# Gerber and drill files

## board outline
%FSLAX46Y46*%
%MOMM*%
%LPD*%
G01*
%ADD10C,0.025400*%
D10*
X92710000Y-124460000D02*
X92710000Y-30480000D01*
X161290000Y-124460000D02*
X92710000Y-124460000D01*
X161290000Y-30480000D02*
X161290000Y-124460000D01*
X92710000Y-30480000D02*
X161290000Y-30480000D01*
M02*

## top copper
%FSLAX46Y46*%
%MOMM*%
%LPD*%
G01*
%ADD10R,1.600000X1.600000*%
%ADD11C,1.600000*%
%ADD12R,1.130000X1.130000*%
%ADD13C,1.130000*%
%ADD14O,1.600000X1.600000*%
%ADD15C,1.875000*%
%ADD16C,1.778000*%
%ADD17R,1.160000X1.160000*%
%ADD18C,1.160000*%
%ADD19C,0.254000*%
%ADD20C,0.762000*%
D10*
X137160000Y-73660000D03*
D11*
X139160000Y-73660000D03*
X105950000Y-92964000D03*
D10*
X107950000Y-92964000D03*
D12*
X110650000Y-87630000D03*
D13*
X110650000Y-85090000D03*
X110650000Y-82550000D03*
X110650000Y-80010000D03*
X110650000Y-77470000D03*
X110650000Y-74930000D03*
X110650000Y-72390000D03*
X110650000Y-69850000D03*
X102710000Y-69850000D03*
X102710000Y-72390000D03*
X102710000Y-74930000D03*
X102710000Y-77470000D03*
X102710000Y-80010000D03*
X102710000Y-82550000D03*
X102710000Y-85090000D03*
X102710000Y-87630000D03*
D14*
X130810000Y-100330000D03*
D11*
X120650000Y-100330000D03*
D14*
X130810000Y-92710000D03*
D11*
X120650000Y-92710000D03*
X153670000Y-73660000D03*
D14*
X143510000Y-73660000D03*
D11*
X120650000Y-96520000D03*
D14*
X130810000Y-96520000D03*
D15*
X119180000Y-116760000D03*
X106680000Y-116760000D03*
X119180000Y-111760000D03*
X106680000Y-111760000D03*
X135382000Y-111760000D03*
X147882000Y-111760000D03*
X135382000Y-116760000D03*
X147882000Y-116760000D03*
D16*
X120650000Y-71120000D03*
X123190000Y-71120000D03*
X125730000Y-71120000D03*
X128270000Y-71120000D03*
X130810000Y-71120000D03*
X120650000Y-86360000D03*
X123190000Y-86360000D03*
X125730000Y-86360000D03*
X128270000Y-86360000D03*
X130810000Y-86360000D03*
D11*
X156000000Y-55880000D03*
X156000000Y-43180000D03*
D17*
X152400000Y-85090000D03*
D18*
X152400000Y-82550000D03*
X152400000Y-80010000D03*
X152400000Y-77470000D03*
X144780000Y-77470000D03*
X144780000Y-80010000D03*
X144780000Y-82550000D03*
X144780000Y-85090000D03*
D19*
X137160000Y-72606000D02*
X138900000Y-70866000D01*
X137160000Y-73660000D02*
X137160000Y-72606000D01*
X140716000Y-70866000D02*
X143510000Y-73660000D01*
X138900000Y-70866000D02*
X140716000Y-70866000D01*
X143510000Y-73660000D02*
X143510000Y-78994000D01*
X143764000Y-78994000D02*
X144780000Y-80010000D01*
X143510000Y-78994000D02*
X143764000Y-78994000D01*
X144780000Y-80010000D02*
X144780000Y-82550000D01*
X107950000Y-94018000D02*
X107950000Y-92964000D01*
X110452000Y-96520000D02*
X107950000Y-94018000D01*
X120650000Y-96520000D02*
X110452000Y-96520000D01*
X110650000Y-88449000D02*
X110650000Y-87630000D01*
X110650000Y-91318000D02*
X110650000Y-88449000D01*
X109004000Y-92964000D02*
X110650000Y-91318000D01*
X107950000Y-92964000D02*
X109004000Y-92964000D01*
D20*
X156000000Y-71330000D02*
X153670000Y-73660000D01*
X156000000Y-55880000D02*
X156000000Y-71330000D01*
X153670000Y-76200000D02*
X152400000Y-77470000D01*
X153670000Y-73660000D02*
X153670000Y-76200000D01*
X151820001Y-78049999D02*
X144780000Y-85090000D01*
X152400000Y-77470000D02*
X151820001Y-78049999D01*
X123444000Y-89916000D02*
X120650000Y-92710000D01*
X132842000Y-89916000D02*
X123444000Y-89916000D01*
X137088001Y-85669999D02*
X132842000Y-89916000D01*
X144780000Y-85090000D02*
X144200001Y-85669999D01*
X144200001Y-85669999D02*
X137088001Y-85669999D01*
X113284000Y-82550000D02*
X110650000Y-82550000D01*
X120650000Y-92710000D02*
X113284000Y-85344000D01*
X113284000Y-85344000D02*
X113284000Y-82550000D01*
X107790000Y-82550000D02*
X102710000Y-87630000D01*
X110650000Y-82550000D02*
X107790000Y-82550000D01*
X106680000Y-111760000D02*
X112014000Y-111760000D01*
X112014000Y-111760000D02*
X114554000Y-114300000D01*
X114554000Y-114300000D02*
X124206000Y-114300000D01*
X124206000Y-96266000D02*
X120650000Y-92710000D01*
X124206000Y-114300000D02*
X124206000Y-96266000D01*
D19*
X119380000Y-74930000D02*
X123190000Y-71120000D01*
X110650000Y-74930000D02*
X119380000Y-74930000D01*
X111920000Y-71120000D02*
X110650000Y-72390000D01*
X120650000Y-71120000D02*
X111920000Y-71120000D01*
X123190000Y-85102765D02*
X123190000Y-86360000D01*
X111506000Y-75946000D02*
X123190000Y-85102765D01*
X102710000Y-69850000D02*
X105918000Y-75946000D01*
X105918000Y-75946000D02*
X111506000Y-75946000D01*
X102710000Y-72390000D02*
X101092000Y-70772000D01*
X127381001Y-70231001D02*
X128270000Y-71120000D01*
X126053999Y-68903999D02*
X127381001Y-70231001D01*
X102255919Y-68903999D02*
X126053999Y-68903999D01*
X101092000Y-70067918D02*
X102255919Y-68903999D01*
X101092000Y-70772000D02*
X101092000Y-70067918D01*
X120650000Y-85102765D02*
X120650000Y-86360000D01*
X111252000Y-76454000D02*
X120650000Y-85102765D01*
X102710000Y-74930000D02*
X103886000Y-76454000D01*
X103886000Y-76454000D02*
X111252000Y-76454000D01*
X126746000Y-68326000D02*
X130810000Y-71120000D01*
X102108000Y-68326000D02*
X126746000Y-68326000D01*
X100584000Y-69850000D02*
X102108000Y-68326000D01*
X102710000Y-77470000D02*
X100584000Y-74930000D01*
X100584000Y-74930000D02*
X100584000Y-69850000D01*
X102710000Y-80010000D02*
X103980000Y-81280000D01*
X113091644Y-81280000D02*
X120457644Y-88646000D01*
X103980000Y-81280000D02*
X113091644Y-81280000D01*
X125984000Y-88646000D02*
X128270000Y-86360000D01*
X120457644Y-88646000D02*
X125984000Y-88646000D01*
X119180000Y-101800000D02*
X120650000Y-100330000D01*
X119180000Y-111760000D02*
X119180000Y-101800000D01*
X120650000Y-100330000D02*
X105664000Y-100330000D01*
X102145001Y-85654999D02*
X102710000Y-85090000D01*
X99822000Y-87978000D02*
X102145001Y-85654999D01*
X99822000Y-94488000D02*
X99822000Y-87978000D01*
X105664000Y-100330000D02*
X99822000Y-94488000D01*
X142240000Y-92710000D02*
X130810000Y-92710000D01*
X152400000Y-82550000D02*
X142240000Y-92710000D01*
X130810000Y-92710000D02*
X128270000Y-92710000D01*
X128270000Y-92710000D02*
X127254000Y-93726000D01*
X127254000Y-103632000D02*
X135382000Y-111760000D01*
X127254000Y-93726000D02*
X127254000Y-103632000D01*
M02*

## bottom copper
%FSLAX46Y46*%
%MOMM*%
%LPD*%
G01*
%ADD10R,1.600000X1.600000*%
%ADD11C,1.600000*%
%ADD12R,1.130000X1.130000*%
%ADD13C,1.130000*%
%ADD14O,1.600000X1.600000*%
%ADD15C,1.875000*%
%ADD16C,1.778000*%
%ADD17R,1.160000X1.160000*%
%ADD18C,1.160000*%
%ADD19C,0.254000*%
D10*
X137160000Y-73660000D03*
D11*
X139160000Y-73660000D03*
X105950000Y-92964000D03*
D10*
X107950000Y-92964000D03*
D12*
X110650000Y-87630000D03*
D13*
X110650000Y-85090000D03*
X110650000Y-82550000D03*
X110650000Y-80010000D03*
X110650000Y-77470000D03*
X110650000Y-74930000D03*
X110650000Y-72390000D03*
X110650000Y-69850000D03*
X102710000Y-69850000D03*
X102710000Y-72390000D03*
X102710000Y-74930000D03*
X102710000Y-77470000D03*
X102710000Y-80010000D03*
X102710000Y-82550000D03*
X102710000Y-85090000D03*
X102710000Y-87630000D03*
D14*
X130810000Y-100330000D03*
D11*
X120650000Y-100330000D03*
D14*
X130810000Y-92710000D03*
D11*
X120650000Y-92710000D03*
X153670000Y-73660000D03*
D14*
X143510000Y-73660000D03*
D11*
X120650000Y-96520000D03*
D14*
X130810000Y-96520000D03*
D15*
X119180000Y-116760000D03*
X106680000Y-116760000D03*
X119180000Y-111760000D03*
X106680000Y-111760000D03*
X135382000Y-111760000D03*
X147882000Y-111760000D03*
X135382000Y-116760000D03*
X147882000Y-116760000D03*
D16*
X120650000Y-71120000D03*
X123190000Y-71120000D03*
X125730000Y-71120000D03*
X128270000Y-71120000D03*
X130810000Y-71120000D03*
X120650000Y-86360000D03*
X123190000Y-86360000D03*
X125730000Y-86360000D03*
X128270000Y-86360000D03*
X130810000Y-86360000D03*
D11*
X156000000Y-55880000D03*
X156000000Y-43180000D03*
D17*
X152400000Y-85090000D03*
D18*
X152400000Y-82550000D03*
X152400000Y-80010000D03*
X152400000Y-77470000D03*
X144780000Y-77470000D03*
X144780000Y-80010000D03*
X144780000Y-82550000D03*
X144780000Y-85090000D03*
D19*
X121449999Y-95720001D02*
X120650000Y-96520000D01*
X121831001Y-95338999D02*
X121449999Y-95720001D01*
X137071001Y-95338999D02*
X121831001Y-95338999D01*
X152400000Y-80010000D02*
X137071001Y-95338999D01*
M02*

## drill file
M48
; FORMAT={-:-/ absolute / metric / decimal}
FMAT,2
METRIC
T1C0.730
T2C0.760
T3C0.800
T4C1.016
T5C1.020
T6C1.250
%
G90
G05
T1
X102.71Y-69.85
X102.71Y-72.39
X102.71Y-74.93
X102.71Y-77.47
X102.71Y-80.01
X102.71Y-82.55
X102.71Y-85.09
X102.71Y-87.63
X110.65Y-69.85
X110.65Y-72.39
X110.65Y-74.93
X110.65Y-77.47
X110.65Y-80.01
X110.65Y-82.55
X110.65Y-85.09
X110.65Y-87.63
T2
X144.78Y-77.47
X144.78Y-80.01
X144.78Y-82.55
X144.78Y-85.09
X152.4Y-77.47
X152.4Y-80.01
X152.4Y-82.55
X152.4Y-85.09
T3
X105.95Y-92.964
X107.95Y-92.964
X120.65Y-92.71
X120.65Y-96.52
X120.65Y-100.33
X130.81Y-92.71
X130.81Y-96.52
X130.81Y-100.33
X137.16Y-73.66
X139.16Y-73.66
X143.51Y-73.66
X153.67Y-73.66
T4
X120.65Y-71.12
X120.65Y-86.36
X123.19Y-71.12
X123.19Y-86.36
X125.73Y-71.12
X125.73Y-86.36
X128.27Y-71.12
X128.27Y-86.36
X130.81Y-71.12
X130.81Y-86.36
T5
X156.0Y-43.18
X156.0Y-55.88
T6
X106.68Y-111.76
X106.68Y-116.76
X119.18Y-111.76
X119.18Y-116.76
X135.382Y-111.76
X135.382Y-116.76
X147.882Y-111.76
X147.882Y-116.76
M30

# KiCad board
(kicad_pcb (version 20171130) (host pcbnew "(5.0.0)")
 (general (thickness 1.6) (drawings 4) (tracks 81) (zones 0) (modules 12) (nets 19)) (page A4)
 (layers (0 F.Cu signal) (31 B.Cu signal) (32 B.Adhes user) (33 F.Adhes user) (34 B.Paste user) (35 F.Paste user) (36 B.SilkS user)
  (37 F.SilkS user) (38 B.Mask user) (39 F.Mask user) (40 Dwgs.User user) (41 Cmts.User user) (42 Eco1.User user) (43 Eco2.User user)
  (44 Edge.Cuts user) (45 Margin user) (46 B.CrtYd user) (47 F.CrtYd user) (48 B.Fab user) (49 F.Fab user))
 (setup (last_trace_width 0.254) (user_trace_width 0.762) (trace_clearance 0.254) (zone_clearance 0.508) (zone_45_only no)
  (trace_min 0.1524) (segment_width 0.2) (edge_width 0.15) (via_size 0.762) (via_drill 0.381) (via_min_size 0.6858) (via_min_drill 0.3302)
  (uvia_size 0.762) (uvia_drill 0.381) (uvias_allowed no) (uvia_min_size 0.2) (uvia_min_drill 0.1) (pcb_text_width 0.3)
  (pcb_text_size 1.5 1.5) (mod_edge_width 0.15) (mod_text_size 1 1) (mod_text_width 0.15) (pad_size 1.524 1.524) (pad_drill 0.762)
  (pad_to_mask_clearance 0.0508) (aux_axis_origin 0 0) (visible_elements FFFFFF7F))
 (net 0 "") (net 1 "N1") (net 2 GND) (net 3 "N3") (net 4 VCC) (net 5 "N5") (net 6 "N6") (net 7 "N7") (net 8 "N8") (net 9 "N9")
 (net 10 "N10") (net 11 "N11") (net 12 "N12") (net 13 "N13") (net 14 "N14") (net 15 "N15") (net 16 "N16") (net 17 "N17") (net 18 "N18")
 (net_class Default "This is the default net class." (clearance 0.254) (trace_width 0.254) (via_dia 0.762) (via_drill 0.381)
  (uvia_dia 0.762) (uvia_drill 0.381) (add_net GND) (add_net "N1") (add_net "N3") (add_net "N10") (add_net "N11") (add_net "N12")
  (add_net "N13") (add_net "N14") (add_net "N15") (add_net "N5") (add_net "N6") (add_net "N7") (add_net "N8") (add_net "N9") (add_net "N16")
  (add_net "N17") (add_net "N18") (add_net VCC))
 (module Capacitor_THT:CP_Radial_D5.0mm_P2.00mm (layer F.Cu) (at 137.16 73.66)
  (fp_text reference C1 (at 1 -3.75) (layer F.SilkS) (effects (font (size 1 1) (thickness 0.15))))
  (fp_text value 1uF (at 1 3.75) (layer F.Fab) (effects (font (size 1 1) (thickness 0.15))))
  (pad 1 thru_hole rect (at 0 0) (size 1.6 1.6) (drill 0.8) (layers *.Cu *.Mask) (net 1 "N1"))
  (pad 2 thru_hole circle (at 2 0) (size 1.6 1.6) (drill 0.8) (layers *.Cu *.Mask) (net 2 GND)))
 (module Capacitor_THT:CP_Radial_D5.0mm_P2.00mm (layer F.Cu) (at 107.95 92.964 180)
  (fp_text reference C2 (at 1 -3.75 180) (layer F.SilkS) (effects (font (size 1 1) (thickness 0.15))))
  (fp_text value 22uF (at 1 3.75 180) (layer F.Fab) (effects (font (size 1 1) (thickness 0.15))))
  (pad 2 thru_hole circle (at 2 0 180) (size 1.6 1.6) (drill 0.8) (layers *.Cu *.Mask) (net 2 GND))
  (pad 1 thru_hole rect (at 0 0 180) (size 1.6 1.6) (drill 0.8) (layers *.Cu *.Mask) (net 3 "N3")))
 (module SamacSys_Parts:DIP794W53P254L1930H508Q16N (layer F.Cu) (at 106.68 78.74 180)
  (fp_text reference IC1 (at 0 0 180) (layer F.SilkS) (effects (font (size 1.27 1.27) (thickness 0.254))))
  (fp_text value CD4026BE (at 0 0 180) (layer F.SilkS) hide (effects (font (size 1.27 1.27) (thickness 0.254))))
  (pad 1 thru_hole rect (at -3.97 -8.89 180) (size 1.13 1.13) (drill 0.73) (layers *.Cu *.Mask) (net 3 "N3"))
  (pad 2 thru_hole circle (at -3.97 -6.35 180) (size 1.13 1.13) (drill 0.73) (layers *.Cu *.Mask) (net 2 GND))
  (pad 3 thru_hole circle (at -3.97 -3.81 180) (size 1.13 1.13) (drill 0.73) (layers *.Cu *.Mask) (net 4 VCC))
  (pad 4 thru_hole circle (at -3.97 -1.27 180) (size 1.13 1.13) (drill 0.73) (layers *.Cu *.Mask) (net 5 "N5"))
  (pad 5 thru_hole circle (at -3.97 1.27 180) (size 1.13 1.13) (drill 0.73) (layers *.Cu *.Mask) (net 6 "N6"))
  (pad 6 thru_hole circle (at -3.97 3.81 180) (size 1.13 1.13) (drill 0.73) (layers *.Cu *.Mask) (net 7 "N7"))
  (pad 7 thru_hole circle (at -3.97 6.35 180) (size 1.13 1.13) (drill 0.73) (layers *.Cu *.Mask) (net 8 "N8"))
  (pad 8 thru_hole circle (at -3.97 8.89 180) (size 1.13 1.13) (drill 0.73) (layers *.Cu *.Mask) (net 2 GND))
  (pad 9 thru_hole circle (at 3.97 8.89 180) (size 1.13 1.13) (drill 0.73) (layers *.Cu *.Mask) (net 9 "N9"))
  (pad 10 thru_hole circle (at 3.97 6.35 180) (size 1.13 1.13) (drill 0.73) (layers *.Cu *.Mask) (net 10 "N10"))
  (pad 11 thru_hole circle (at 3.97 3.81 180) (size 1.13 1.13) (drill 0.73) (layers *.Cu *.Mask) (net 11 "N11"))
  (pad 12 thru_hole circle (at 3.97 1.27 180) (size 1.13 1.13) (drill 0.73) (layers *.Cu *.Mask) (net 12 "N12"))
  (pad 13 thru_hole circle (at 3.97 -1.27 180) (size 1.13 1.13) (drill 0.73) (layers *.Cu *.Mask) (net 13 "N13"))
  (pad 14 thru_hole circle (at 3.97 -3.81 180) (size 1.13 1.13) (drill 0.73) (layers *.Cu *.Mask) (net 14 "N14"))
  (pad 15 thru_hole circle (at 3.97 -6.35 180) (size 1.13 1.13) (drill 0.73) (layers *.Cu *.Mask) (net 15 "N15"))
  (pad 16 thru_hole circle (at 3.97 -8.89 180) (size 1.13 1.13) (drill 0.73) (layers *.Cu *.Mask) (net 4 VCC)))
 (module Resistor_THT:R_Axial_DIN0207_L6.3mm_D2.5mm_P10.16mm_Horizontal (layer F.Cu) (at 120.65 100.33)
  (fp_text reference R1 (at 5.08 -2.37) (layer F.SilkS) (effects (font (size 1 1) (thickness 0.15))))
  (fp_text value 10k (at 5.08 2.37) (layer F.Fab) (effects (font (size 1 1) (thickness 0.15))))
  (pad 2 thru_hole oval (at 10.16 0) (size 1.6 1.6) (drill 0.8) (layers *.Cu *.Mask) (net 2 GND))
  (pad 1 thru_hole circle (at 0 0) (size 1.6 1.6) (drill 0.8) (layers *.Cu *.Mask) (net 15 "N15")))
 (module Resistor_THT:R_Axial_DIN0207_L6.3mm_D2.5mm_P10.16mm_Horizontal (layer F.Cu) (at 120.65 92.71)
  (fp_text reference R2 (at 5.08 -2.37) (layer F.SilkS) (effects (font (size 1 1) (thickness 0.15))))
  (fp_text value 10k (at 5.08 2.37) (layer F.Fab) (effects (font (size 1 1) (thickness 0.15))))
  (pad 2 thru_hole oval (at 10.16 0) (size 1.6 1.6) (drill 0.8) (layers *.Cu *.Mask) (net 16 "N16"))
  (pad 1 thru_hole circle (at 0 0) (size 1.6 1.6) (drill 0.8) (layers *.Cu *.Mask) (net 4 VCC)))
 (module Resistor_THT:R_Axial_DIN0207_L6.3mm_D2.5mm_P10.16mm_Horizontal (layer F.Cu) (at 153.67 73.66 180)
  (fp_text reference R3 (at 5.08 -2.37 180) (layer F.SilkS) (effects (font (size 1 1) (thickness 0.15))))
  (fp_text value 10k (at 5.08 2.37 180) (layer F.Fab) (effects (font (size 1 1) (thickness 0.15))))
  (pad 1 thru_hole circle (at 0 0 180) (size 1.6 1.6) (drill 0.8) (layers *.Cu *.Mask) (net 4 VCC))
  (pad 2 thru_hole oval (at 10.16 0 180) (size 1.6 1.6) (drill 0.8) (layers *.Cu *.Mask) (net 1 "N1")))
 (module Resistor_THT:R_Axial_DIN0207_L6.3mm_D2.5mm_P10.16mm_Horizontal (layer F.Cu) (at 120.65 96.52)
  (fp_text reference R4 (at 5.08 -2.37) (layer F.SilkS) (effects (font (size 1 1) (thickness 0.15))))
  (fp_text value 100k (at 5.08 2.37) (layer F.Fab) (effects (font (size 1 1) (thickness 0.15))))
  (pad 1 thru_hole circle (at 0 0) (size 1.6 1.6) (drill 0.8) (layers *.Cu *.Mask) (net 3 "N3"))
  (pad 2 thru_hole oval (at 10.16 0) (size 1.6 1.6) (drill 0.8) (layers *.Cu *.Mask) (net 2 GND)))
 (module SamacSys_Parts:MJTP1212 (layer F.Cu) (at 106.68 111.76)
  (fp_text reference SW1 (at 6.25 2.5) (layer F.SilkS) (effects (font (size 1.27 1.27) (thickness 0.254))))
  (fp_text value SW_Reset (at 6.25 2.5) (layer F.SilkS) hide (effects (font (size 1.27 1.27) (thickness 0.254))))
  (pad 4 thru_hole circle (at 12.5 5) (size 1.875 1.875) (drill 1.25) (layers *.Cu *.Mask))
  (pad 3 thru_hole circle (at 0 5) (size 1.875 1.875) (drill 1.25) (layers *.Cu *.Mask))
  (pad 2 thru_hole circle (at 12.5 0) (size 1.875 1.875) (drill 1.25) (layers *.Cu *.Mask) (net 15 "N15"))
  (pad 1 thru_hole circle (at 0 0) (size 1.875 1.875) (drill 1.25) (layers *.Cu *.Mask) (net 4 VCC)))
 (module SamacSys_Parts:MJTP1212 (layer F.Cu) (at 135.382 111.76)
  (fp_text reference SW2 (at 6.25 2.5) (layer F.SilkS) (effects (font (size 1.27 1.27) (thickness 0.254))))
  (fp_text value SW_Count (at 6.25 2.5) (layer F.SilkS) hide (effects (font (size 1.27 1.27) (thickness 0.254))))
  (pad 1 thru_hole circle (at 0 0) (size 1.875 1.875) (drill 1.25) (layers *.Cu *.Mask) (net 16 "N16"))
  (pad 2 thru_hole circle (at 12.5 0) (size 1.875 1.875) (drill 1.25) (layers *.Cu *.Mask) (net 2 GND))
  (pad 3 thru_hole circle (at 0 5) (size 1.875 1.875) (drill 1.25) (layers *.Cu *.Mask))
  (pad 4 thru_hole circle (at 12.5 5) (size 1.875 1.875) (drill 1.25) (layers *.Cu *.Mask)))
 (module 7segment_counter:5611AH (layer F.Cu) (at 125.73 78.74)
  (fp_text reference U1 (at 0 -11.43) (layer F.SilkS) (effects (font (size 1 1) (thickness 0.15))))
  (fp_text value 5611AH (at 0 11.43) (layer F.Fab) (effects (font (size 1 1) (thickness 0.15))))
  (pad 1 thru_hole circle (at -5.08 -7.62) (size 1.778 1.778) (drill 1.016) (layers *.Cu *.Mask) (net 8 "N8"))
  (pad 2 thru_hole circle (at -2.54 -7.62) (size 1.778 1.778) (drill 1.016) (layers *.Cu *.Mask) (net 7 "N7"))
  (pad 3 thru_hole circle (at 0 -7.62) (size 1.778 1.778) (drill 1.016) (layers *.Cu *.Mask) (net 2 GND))
  (pad 4 thru_hole circle (at 2.54 -7.62) (size 1.778 1.778) (drill 1.016) (layers *.Cu *.Mask) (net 10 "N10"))
  (pad 5 thru_hole circle (at 5.08 -7.62) (size 1.778 1.778) (drill 1.016) (layers *.Cu *.Mask) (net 12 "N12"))
  (pad 6 thru_hole circle (at -5.08 7.62) (size 1.778 1.778) (drill 1.016) (layers *.Cu *.Mask) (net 11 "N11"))
  (pad 7 thru_hole circle (at -2.54 7.62) (size 1.778 1.778) (drill 1.016) (layers *.Cu *.Mask) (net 9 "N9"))
  (pad 8 thru_hole circle (at 0 7.62) (size 1.778 1.778) (drill 1.016) (layers *.Cu *.Mask) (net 2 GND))
  (pad 9 thru_hole circle (at 2.54 7.62) (size 1.778 1.778) (drill 1.016) (layers *.Cu *.Mask) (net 13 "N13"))
  (pad 10 thru_hole circle (at 5.08 7.62) (size 1.778 1.778) (drill 1.016) (layers *.Cu *.Mask) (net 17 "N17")))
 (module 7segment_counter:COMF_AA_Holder (layer F.Cu) (at 127 49.53)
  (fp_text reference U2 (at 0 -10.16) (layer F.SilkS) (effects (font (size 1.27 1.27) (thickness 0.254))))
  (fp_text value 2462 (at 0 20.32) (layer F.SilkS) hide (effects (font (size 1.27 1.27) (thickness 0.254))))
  (pad 1 thru_hole circle (at 29 6.35) (size 1.6 1.6) (drill 1.02) (layers *.Cu *.Mask) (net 4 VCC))
  (pad 2 thru_hole circle (at 29 -6.35) (size 1.6 1.6) (drill 1.02) (layers *.Cu *.Mask) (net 2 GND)))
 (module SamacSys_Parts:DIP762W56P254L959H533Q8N (layer F.Cu) (at 148.59 81.28 180)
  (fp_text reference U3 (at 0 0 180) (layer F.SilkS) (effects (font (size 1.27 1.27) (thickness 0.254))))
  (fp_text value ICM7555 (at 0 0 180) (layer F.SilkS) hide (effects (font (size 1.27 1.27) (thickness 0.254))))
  (pad 1 thru_hole rect (at -3.81 -3.81 180) (size 1.16 1.16) (drill 0.76) (layers *.Cu *.Mask) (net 2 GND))
  (pad 2 thru_hole circle (at -3.81 -1.27 180) (size 1.16 1.16) (drill 0.76) (layers *.Cu *.Mask) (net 16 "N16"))
  (pad 3 thru_hole circle (at -3.81 1.27 180) (size 1.16 1.16) (drill 0.76) (layers *.Cu *.Mask) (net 3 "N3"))
  (pad 4 thru_hole circle (at -3.81 3.81 180) (size 1.16 1.16) (drill 0.76) (layers *.Cu *.Mask) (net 4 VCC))
  (pad 5 thru_hole circle (at 3.81 3.81 180) (size 1.16 1.16) (drill 0.76) (layers *.Cu *.Mask) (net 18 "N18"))
  (pad 6 thru_hole circle (at 3.81 1.27 180) (size 1.16 1.16) (drill 0.76) (layers *.Cu *.Mask) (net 1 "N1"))
  (pad 7 thru_hole circle (at 3.81 -1.27 180) (size 1.16 1.16) (drill 0.76) (layers *.Cu *.Mask) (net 1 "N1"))
  (pad 8 thru_hole circle (at 3.81 -3.81 180) (size 1.16 1.16) (drill 0.76) (layers *.Cu *.Mask) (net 4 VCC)))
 (gr_line (start 92.71 124.46) (end 92.71 30.48) (layer Edge.Cuts) (width 0.0254))
 (gr_line (start 161.29 124.46) (end 92.71 124.46) (layer Edge.Cuts) (width 0.0254))
 (gr_line (start 161.29 30.48) (end 161.29 124.46) (layer Edge.Cuts) (width 0.0254))
 (gr_line (start 92.71 30.48) (end 161.29 30.48) (layer Edge.Cuts) (width 0.0254))
 (segment (start 137.16 72.606) (end 138.9 70.866) (width 0.254) (layer F.Cu) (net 1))
 (segment (start 137.16 73.66) (end 137.16 72.606) (width 0.254) (layer F.Cu) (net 1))
 (segment (start 140.716 70.866) (end 143.51 73.66) (width 0.254) (layer F.Cu) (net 1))
 (segment (start 138.9 70.866) (end 140.716 70.866) (width 0.254) (layer F.Cu) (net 1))
 (segment (start 143.51 73.66) (end 143.51 78.994) (width 0.254) (layer F.Cu) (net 1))
 (segment (start 143.764 78.994) (end 144.78 80.01) (width 0.254) (layer F.Cu) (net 1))
 (segment (start 143.51 78.994) (end 143.764 78.994) (width 0.254) (layer F.Cu) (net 1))
 (segment (start 144.78 80.01) (end 144.78 82.55) (width 0.254) (layer F.Cu) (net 1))
 (segment (start 107.95 94.018) (end 107.95 92.964) (width 0.254) (layer F.Cu) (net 3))
 (segment (start 110.452 96.52) (end 107.95 94.018) (width 0.254) (layer F.Cu) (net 3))
 (segment (start 120.65 96.52) (end 110.452 96.52) (width 0.254) (layer F.Cu) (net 3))
 (segment (start 121.449999 95.720001) (end 120.65 96.52) (width 0.254) (layer B.Cu) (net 3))
 (segment (start 121.831001 95.338999) (end 121.449999 95.720001) (width 0.254) (layer B.Cu) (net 3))
 (segment (start 137.071001 95.338999) (end 121.831001 95.338999) (width 0.254) (layer B.Cu) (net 3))
 (segment (start 152.4 80.01) (end 137.071001 95.338999) (width 0.254) (layer B.Cu) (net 3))
 (segment (start 110.65 88.449) (end 110.65 87.63) (width 0.254) (layer F.Cu) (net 3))
 (segment (start 110.65 91.318) (end 110.65 88.449) (width 0.254) (layer F.Cu) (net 3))
 (segment (start 109.004 92.964) (end 110.65 91.318) (width 0.254) (layer F.Cu) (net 3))
 (segment (start 107.95 92.964) (end 109.004 92.964) (width 0.254) (layer F.Cu) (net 3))
 (segment (start 156 71.33) (end 153.67 73.66) (width 0.762) (layer F.Cu) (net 4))
 (segment (start 156 55.88) (end 156 71.33) (width 0.762) (layer F.Cu) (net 4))
 (segment (start 153.67 76.2) (end 152.4 77.47) (width 0.762) (layer F.Cu) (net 4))
 (segment (start 153.67 73.66) (end 153.67 76.2) (width 0.762) (layer F.Cu) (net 4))
 (segment (start 151.820001 78.049999) (end 144.78 85.09) (width 0.762) (layer F.Cu) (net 4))
 (segment (start 152.4 77.47) (end 151.820001 78.049999) (width 0.762) (layer F.Cu) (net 4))
 (segment (start 123.444 89.916) (end 120.65 92.71) (width 0.762) (layer F.Cu) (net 4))
 (segment (start 132.842 89.916) (end 123.444 89.916) (width 0.762) (layer F.Cu) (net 4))
 (segment (start 137.088001 85.669999) (end 132.842 89.916) (width 0.762) (layer F.Cu) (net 4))
 (segment (start 144.78 85.09) (end 144.200001 85.669999) (width 0.762) (layer F.Cu) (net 4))
 (segment (start 144.200001 85.669999) (end 137.088001 85.669999) (width 0.762) (layer F.Cu) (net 4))
 (segment (start 113.284 82.55) (end 110.65 82.55) (width 0.762) (layer F.Cu) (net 4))
 (segment (start 120.65 92.71) (end 113.284 85.344) (width 0.762) (layer F.Cu) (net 4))
 (segment (start 113.284 85.344) (end 113.284 82.55) (width 0.762) (layer F.Cu) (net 4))
 (segment (start 107.79 82.55) (end 102.71 87.63) (width 0.762) (layer F.Cu) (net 4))
 (segment (start 110.65 82.55) (end 107.79 82.55) (width 0.762) (layer F.Cu) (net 4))
 (segment (start 106.68 111.76) (end 112.014 111.76) (width 0.762) (layer F.Cu) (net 4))
 (segment (start 112.014 111.76) (end 114.554 114.3) (width 0.762) (layer F.Cu) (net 4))
 (segment (start 114.554 114.3) (end 124.206 114.3) (width 0.762) (layer F.Cu) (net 4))
 (segment (start 124.206 96.266) (end 120.65 92.71) (width 0.762) (layer F.Cu) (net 4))
 (segment (start 124.206 114.3) (end 124.206 96.266) (width 0.762) (layer F.Cu) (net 4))
 (segment (start 119.38 74.93) (end 123.19 71.12) (width 0.254) (layer F.Cu) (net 7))
 (segment (start 110.65 74.93) (end 119.38 74.93) (width 0.254) (layer F.Cu) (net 7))
 (segment (start 111.92 71.12) (end 110.65 72.39) (width 0.254) (layer F.Cu) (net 8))
 (segment (start 120.65 71.12) (end 111.92 71.12) (width 0.254) (layer F.Cu) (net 8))
 (segment (start 123.19 85.102765) (end 123.19 86.36) (width 0.254) (layer F.Cu) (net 9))
 (segment (start 111.506 75.946) (end 123.19 85.102765) (width 0.254) (layer F.Cu) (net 9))
 (segment (start 102.71 69.85) (end 105.918 75.946) (width 0.254) (layer F.Cu) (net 9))
 (segment (start 105.918 75.946) (end 111.506 75.946) (width 0.254) (layer F.Cu) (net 9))
 (segment (start 102.71 72.39) (end 101.092 70.772) (width 0.254) (layer F.Cu) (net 10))
 (segment (start 127.381001 70.231001) (end 128.27 71.12) (width 0.254) (layer F.Cu) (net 10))
 (segment (start 126.053999 68.903999) (end 127.381001 70.231001) (width 0.254) (layer F.Cu) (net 10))
 (segment (start 102.255919 68.903999) (end 126.053999 68.903999) (width 0.254) (layer F.Cu) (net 10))
 (segment (start 101.092 70.067918) (end 102.255919 68.903999) (width 0.254) (layer F.Cu) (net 10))
 (segment (start 101.092 70.772) (end 101.092 70.067918) (width 0.254) (layer F.Cu) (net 10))
 (segment (start 120.65 85.102765) (end 120.65 86.36) (width 0.254) (layer F.Cu) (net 11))
 (segment (start 111.252 76.454) (end 120.65 85.102765) (width 0.254) (layer F.Cu) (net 11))
 (segment (start 102.71 74.93) (end 103.886 76.454) (width 0.254) (layer F.Cu) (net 11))
 (segment (start 103.886 76.454) (end 111.252 76.454) (width 0.254) (layer F.Cu) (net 11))
 (segment (start 126.746 68.326) (end 130.81 71.12) (width 0.254) (layer F.Cu) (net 12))
 (segment (start 102.108 68.326) (end 126.746 68.326) (width 0.254) (layer F.Cu) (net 12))
 (segment (start 100.584 69.85) (end 102.108 68.326) (width 0.254) (layer F.Cu) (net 12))
 (segment (start 102.71 77.47) (end 100.584 74.93) (width 0.254) (layer F.Cu) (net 12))
 (segment (start 100.584 74.93) (end 100.584 69.85) (width 0.254) (layer F.Cu) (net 12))
 (segment (start 102.71 80.01) (end 103.98 81.28) (width 0.254) (layer F.Cu) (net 13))
 (segment (start 113.091644 81.28) (end 120.457644 88.646) (width 0.254) (layer F.Cu) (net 13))
 (segment (start 103.98 81.28) (end 113.091644 81.28) (width 0.254) (layer F.Cu) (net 13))
 (segment (start 125.984 88.646) (end 128.27 86.36) (width 0.254) (layer F.Cu) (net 13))
 (segment (start 120.457644 88.646) (end 125.984 88.646) (width 0.254) (layer F.Cu) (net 13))
 (segment (start 119.18 101.8) (end 120.65 100.33) (width 0.254) (layer F.Cu) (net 15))
 (segment (start 119.18 111.76) (end 119.18 101.8) (width 0.254) (layer F.Cu) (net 15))
 (segment (start 120.65 100.33) (end 105.664 100.33) (width 0.254) (layer F.Cu) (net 15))
 (segment (start 102.145001 85.654999) (end 102.71 85.09) (width 0.254) (layer F.Cu) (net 15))
 (segment (start 99.822 87.978) (end 102.145001 85.654999) (width 0.254) (layer F.Cu) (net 15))
 (segment (start 99.822 94.488) (end 99.822 87.978) (width 0.254) (layer F.Cu) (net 15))
 (segment (start 105.664 100.33) (end 99.822 94.488) (width 0.254) (layer F.Cu) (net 15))
 (segment (start 142.24 92.71) (end 130.81 92.71) (width 0.254) (layer F.Cu) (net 16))
 (segment (start 152.4 82.55) (end 142.24 92.71) (width 0.254) (layer F.Cu) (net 16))
 (segment (start 130.81 92.71) (end 128.27 92.71) (width 0.254) (layer F.Cu) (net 16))
 (segment (start 128.27 92.71) (end 127.254 93.726) (width 0.254) (layer F.Cu) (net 16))
 (segment (start 127.254 103.632) (end 135.382 111.76) (width 0.254) (layer F.Cu) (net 16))
 (segment (start 127.254 93.726) (end 127.254 103.632) (width 0.254) (layer F.Cu) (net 16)))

